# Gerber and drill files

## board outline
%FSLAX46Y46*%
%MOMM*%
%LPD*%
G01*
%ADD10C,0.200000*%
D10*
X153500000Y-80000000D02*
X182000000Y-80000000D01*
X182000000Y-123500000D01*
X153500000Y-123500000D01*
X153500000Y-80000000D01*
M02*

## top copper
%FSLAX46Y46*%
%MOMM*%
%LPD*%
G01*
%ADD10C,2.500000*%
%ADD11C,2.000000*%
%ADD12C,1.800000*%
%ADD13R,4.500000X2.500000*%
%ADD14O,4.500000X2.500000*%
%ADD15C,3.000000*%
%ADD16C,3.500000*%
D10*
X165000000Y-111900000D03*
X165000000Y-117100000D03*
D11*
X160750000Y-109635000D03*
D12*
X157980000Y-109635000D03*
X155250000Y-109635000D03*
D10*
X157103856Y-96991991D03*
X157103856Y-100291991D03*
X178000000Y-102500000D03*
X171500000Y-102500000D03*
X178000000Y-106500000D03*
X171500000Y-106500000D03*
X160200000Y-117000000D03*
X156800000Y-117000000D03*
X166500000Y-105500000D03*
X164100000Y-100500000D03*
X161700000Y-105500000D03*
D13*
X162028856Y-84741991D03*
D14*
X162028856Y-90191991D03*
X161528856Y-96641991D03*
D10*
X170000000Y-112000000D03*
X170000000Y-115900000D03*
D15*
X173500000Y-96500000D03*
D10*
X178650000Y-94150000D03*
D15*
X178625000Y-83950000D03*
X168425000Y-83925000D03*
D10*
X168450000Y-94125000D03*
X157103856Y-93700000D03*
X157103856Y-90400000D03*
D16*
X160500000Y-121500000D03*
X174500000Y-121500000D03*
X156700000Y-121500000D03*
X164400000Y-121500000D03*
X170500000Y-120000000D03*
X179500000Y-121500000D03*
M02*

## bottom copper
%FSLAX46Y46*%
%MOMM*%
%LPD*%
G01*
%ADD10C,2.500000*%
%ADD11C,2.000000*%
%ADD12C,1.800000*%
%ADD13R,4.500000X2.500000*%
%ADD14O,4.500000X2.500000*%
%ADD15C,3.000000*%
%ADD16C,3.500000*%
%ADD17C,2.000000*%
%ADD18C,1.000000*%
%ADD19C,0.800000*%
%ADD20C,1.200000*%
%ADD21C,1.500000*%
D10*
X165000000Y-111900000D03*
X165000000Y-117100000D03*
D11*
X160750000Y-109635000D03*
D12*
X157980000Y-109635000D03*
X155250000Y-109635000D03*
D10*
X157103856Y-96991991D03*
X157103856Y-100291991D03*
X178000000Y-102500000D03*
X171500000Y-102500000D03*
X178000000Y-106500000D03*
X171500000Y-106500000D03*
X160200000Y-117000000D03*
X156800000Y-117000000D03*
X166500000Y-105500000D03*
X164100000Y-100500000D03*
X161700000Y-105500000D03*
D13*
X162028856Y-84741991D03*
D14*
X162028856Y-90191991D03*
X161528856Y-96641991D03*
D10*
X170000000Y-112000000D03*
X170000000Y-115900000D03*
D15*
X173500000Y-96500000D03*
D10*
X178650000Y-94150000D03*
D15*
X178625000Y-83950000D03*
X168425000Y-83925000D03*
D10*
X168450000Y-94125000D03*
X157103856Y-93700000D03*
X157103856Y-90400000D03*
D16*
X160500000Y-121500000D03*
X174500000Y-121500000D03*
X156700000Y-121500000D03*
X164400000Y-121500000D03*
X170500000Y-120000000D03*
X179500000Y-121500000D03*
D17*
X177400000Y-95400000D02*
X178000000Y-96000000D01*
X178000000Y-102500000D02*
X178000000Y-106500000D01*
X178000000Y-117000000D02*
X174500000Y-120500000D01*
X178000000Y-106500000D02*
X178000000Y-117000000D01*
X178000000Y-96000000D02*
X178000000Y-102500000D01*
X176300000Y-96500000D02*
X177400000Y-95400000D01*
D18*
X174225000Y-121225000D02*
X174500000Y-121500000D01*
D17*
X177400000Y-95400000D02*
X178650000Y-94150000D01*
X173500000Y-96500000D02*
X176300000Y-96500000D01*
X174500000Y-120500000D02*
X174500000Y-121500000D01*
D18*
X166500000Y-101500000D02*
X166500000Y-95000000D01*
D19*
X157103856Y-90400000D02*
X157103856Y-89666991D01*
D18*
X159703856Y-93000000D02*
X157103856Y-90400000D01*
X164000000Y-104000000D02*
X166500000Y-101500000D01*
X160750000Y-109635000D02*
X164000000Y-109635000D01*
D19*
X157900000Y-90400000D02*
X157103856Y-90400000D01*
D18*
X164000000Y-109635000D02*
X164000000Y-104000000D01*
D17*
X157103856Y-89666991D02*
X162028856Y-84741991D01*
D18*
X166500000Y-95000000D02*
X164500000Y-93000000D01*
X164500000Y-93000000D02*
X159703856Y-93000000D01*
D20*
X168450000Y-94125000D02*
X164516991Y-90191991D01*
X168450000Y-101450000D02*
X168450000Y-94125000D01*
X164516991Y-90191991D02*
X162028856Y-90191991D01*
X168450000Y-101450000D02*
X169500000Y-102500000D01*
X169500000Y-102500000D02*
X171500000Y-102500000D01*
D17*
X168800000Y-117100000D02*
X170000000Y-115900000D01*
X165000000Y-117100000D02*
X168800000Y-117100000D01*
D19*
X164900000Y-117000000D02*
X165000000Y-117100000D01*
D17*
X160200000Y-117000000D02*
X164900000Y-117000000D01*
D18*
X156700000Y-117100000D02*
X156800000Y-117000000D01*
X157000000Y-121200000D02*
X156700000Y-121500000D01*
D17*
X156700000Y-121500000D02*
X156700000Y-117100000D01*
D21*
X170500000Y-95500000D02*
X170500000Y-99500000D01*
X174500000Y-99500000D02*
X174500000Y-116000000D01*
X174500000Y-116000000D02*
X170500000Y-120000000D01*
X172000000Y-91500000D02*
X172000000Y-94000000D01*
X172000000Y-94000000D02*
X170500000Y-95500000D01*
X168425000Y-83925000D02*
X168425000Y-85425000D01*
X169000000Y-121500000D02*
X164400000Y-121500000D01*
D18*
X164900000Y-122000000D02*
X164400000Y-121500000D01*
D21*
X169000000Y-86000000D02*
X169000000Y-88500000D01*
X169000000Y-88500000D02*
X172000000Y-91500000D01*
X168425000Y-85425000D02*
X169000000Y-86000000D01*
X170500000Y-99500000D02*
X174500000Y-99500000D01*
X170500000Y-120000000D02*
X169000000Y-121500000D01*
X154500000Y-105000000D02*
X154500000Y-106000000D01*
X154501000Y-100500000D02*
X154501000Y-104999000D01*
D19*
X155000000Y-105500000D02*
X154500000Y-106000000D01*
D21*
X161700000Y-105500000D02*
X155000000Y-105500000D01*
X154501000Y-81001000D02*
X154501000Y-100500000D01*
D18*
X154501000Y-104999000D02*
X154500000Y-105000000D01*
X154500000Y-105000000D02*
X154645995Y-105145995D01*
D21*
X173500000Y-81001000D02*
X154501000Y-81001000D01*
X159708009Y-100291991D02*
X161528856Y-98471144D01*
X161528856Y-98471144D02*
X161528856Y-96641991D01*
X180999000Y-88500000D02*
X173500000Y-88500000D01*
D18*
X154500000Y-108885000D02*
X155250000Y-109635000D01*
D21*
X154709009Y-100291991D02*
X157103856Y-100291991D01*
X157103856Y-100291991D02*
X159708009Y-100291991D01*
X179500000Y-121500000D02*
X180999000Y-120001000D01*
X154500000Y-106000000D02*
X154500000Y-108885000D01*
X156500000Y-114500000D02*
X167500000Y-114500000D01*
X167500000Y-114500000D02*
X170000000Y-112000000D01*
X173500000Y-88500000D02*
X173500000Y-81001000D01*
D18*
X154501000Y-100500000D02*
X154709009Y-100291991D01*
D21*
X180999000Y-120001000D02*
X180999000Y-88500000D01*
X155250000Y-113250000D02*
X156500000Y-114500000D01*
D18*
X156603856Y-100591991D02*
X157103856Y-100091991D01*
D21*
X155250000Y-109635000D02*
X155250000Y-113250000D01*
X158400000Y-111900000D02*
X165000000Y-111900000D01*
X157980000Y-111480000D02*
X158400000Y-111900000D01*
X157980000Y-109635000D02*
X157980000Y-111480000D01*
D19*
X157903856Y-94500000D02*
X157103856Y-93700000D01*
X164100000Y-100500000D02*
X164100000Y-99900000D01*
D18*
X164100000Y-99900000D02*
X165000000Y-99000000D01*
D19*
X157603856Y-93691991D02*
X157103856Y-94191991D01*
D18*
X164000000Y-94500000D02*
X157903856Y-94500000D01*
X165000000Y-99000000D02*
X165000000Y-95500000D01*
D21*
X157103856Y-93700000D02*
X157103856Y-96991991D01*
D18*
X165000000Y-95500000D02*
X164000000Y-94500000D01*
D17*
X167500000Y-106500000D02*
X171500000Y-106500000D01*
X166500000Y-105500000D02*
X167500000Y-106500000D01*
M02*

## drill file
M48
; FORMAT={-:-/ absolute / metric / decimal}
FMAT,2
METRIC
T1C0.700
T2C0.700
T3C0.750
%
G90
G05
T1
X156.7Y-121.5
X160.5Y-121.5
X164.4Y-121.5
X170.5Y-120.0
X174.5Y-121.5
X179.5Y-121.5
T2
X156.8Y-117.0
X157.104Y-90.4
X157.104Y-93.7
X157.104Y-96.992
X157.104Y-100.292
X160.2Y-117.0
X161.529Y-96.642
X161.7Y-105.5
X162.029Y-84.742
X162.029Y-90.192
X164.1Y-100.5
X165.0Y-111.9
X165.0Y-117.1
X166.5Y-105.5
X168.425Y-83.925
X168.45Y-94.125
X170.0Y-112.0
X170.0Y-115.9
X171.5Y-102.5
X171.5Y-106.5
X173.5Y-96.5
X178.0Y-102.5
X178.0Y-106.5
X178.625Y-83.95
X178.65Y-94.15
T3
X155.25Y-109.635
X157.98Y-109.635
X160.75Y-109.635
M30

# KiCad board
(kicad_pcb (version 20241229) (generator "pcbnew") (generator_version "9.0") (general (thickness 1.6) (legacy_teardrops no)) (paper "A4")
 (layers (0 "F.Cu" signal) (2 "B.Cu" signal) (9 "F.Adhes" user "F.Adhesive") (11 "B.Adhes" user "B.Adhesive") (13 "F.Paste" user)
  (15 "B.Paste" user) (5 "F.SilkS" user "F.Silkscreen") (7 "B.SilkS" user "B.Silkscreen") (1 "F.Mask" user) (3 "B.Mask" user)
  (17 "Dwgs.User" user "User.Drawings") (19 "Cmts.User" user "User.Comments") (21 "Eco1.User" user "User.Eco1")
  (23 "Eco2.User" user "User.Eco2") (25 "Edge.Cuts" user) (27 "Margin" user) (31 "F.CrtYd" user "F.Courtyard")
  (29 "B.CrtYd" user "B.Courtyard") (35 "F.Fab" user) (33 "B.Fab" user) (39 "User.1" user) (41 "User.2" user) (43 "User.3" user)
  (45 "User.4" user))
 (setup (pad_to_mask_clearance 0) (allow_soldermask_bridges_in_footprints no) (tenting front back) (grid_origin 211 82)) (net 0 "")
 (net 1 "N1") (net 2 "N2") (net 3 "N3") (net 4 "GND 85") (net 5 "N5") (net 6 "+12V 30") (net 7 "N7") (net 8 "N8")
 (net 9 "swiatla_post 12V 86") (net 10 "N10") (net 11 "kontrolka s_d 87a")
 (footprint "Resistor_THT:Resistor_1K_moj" (layer "F.Cu") (at 165 112.5 -90)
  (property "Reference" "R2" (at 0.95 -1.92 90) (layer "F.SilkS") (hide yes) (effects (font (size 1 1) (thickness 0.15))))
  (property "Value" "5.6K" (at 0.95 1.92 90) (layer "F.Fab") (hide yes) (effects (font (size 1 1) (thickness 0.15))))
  (pad "1" thru_hole circle (at -0.6 0 270) (size 2.5 2.5) (drill 0.7) (layers "*.Cu" "*.Mask") (remove_unused_layers no) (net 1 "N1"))
  (pad "2" thru_hole circle (at 4.6 0 270) (size 2.5 2.5) (drill 0.7) (layers "*.Cu" "*.Mask") (remove_unused_layers no) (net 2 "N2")))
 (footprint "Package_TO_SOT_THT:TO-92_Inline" (layer "F.Cu") (at 159.25 109.635 180)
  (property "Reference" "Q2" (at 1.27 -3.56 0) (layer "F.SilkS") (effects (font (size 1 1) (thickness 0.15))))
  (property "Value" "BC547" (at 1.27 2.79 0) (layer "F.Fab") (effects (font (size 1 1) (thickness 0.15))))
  (pad "1" thru_hole circle (at -1.5 0 180) (size 2 2) (drill 0.75) (layers "*.Cu" "*.Mask") (remove_unused_layers no) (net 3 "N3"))
  (pad "2" thru_hole circle (at 1.27 0 180) (size 1.8 1.8) (drill 0.75) (layers "*.Cu" "*.Mask") (remove_unused_layers no) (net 1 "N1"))
  (pad "3" thru_hole circle (at 4 0 180) (size 1.8 1.8) (drill 0.75) (layers "*.Cu" "*.Mask") (remove_unused_layers no) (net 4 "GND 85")))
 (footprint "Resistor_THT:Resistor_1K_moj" (layer "F.Cu") (at 157.103856 98.191991 -90)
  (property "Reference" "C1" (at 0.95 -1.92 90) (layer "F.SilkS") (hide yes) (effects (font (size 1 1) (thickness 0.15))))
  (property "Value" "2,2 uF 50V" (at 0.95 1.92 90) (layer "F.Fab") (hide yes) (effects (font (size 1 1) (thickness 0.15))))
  (pad "1" thru_hole circle (at -1.2 0 270) (size 2.5 2.5) (drill 0.7) (layers "*.Cu" "*.Mask") (remove_unused_layers no) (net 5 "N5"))
  (pad "2" thru_hole circle (at 2.1 0 270) (size 2.5 2.5) (drill 0.7) (layers "*.Cu" "*.Mask") (remove_unused_layers no) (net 4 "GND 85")))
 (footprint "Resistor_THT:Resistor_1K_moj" (layer "F.Cu") (at 177 102.5 180)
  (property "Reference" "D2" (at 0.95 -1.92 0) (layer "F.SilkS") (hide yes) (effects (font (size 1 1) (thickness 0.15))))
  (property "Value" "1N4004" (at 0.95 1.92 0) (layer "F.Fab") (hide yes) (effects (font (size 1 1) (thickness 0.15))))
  (pad "1" thru_hole circle (at -1 0 180) (size 2.5 2.5) (drill 0.7) (layers "*.Cu" "*.Mask") (remove_unused_layers no) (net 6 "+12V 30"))
  (pad "2" thru_hole circle (at 5.5 0 180) (size 2.5 2.5) (drill 0.7) (layers "*.Cu" "*.Mask") (remove_unused_layers no) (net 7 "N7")))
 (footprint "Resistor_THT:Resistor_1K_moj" (layer "F.Cu") (at 177 106.5 180)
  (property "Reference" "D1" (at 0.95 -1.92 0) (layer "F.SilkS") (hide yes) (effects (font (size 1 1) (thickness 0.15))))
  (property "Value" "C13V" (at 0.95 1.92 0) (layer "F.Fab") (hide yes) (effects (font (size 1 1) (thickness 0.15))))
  (pad "1" thru_hole circle (at -1 0 180) (size 2.5 2.5) (drill 0.7) (layers "*.Cu" "*.Mask") (remove_unused_layers no) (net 6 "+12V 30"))
  (pad "2" thru_hole circle (at 5.5 0 180) (size 2.5 2.5) (drill 0.7) (layers "*.Cu" "*.Mask") (remove_unused_layers no) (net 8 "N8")))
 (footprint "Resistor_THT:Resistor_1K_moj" (layer "F.Cu") (at 158 117)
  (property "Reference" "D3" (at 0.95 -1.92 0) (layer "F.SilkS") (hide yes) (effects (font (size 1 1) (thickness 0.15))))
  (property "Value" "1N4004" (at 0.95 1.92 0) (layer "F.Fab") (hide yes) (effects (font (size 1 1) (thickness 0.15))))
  (pad "" thru_hole circle (at 2.2 0) (size 2.5 2.5) (drill 0.7) (layers "*.Cu" "*.Mask") (remove_unused_layers no) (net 2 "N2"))
  (pad "1" thru_hole circle (at -1.2 0) (size 2.5 2.5) (drill 0.7) (layers "*.Cu" "*.Mask") (remove_unused_layers no)
   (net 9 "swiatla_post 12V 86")))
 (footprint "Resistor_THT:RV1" (layer "F.Cu") (at 164 103.5 -90)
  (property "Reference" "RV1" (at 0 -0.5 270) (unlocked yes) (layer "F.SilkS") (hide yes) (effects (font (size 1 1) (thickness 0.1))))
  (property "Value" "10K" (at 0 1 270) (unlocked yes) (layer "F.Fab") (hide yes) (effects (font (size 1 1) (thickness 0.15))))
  (pad "1" thru_hole circle (at 2 -2.5 270) (size 2.5 2.5) (drill 0.7) (layers "*.Cu" "*.Mask") (remove_unused_layers no) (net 8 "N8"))
  (pad "2" thru_hole circle (at -3 -0.1 270) (size 2.5 2.5) (drill 0.7) (layers "*.Cu" "*.Mask") (remove_unused_layers no) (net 5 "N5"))
  (pad "3" thru_hole circle (at 2 2.3 270) (size 2.5 2.5) (drill 0.7) (layers "*.Cu" "*.Mask") (remove_unused_layers no) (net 4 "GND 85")))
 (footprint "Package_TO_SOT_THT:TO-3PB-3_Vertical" (layer "F.Cu") (at 162.028856 84.741991 -90)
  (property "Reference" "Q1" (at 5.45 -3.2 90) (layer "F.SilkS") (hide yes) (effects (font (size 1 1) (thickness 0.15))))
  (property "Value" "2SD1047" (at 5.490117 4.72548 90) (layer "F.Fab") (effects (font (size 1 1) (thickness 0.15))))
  (pad "1" thru_hole rect (at 0 0 270) (size 2.5 4.5) (drill 0.7) (layers "*.Cu" "*.Mask") (remove_unused_layers no) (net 3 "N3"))
  (pad "2" thru_hole oval (at 5.45 0 270) (size 2.5 4.5) (drill 0.7) (layers "*.Cu" "*.Mask") (remove_unused_layers no) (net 7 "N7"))
  (pad "3" thru_hole oval (at 11.9 0.5 270) (size 2.5 4.5) (drill 0.7) (layers "*.Cu" "*.Mask") (remove_unused_layers no) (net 4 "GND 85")))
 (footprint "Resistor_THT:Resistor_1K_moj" (layer "F.Cu") (at 170 113 -90)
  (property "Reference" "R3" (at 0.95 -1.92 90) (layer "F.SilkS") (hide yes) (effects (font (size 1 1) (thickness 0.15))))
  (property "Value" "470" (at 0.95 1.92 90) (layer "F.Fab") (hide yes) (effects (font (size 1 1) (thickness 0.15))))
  (pad "1" thru_hole circle (at -1 0 270) (size 2.5 2.5) (drill 0.7) (layers "*.Cu" "*.Mask") (remove_unused_layers no) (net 4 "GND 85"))
  (pad "2" thru_hole circle (at 2.9 0 270) (size 2.5 2.5) (drill 0.7) (layers "*.Cu" "*.Mask") (remove_unused_layers no) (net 2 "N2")))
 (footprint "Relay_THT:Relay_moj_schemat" (layer "F.Cu") (at 173.5 97.1 90)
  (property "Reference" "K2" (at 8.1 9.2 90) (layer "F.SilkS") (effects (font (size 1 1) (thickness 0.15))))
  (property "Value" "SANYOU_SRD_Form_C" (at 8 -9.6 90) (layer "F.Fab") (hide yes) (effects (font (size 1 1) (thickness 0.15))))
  (pad "1" thru_hole circle (at 0.6 0 180) (size 3 3) (drill 0.7) (layers "*.Cu" "*.Mask") (remove_unused_layers no) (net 6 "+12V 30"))
  (pad "2" thru_hole circle (at 2.95 5.15 180) (size 2.5 2.5) (drill 0.7) (layers "*.Cu" "*.Mask") (remove_unused_layers no)
   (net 6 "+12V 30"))
  (pad "3" thru_hole circle (at 13.15 5.125 180) (size 3 3) (drill 0.7) (layers "*.Cu" "*.Mask") (remove_unused_layers no) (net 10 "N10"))
  (pad "4" thru_hole circle (at 13.175 -5.075 180) (size 3 3) (drill 0.7) (layers "*.Cu" "*.Mask") (remove_unused_layers no)
   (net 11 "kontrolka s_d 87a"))
  (pad "5" thru_hole circle (at 2.975 -5.05 180) (size 2.5 2.5) (drill 0.7) (layers "*.Cu" "*.Mask") (remove_unused_layers no) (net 7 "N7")))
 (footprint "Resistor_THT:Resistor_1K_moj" (layer "F.Cu") (at 157.103856 92.5 90)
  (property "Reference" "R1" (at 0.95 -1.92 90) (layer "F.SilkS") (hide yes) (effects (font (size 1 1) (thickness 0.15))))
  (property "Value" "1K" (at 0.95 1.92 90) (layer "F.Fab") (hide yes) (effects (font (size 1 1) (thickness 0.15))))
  (pad "1" thru_hole circle (at -1.2 0 90) (size 2.5 2.5) (drill 0.7) (layers "*.Cu" "*.Mask") (remove_unused_layers no) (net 5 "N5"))
  (pad "2" thru_hole circle (at 2.1 0 90) (size 2.5 2.5) (drill 0.7) (layers "*.Cu" "*.Mask") (remove_unused_layers no) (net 3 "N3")))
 (gr_rect (start 153.5 80) (end 182 123.5) (stroke (width 0.2) (type solid)) (fill no) (layer "Edge.Cuts"))
 (via (at 160.5 121.5) (size 3.5) (drill 0.7) (layers "F.Cu" "B.Cu") (free yes) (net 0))
 (via (at 174.5 121.5) (size 3.5) (drill 0.7) (layers "F.Cu" "B.Cu") (free yes) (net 6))
 (segment (start 177.4 95.4) (end 178 96) (width 2) (layer "B.Cu") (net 6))
 (segment (start 178 102.5) (end 178 106.5) (width 2) (layer "B.Cu") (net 6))
 (segment (start 178 117) (end 174.5 120.5) (width 2) (layer "B.Cu") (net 6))
 (segment (start 178 106.5) (end 178 117) (width 2) (layer "B.Cu") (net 6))
 (segment (start 178 96) (end 178 102.5) (width 2) (layer "B.Cu") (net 6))
 (segment (start 176.3 96.5) (end 177.4 95.4) (width 2) (layer "B.Cu") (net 6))
 (segment (start 174.225 121.225) (end 174.5 121.5) (width 1) (layer "B.Cu") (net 6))
 (segment (start 177.4 95.4) (end 178.65 94.15) (width 2) (layer "B.Cu") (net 6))
 (segment (start 173.5 96.5) (end 176.3 96.5) (width 2) (layer "B.Cu") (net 6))
 (segment (start 174.5 120.5) (end 174.5 121.5) (width 2) (layer "B.Cu") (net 6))
 (segment (start 166.5 101.5) (end 166.5 95) (width 1) (layer "B.Cu") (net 3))
 (segment (start 157.103856 90.4) (end 157.103856 89.666991) (width 0.8) (layer "B.Cu") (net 3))
 (segment (start 159.703856 93) (end 157.103856 90.4) (width 1) (layer "B.Cu") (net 3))
 (segment (start 164 104) (end 166.5 101.5) (width 1) (layer "B.Cu") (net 3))
 (segment (start 160.75 109.635) (end 164 109.635) (width 1) (layer "B.Cu") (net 3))
 (segment (start 157.9 90.4) (end 157.103856 90.4) (width 0.8) (layer "B.Cu") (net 3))
 (segment (start 164 109.635) (end 164 104) (width 1) (layer "B.Cu") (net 3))
 (segment (start 157.103856 89.666991) (end 162.028856 84.741991) (width 2) (layer "B.Cu") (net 3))
 (segment (start 166.5 95) (end 164.5 93) (width 1) (layer "B.Cu") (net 3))
 (segment (start 164.5 93) (end 159.703856 93) (width 1) (layer "B.Cu") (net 3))
 (segment (start 168.45 94.125) (end 164.516991 90.191991) (width 1.2) (layer "B.Cu") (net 7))
 (segment (start 168.45 101.45) (end 168.45 94.125) (width 1.2) (layer "B.Cu") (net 7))
 (segment (start 164.516991 90.191991) (end 162.028856 90.191991) (width 1.2) (layer "B.Cu") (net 7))
 (segment (start 168.45 101.45) (end 169.5 102.5) (width 1.2) (layer "B.Cu") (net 7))
 (segment (start 169.5 102.5) (end 171.5 102.5) (width 1.2) (layer "B.Cu") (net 7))
 (segment (start 168.8 117.1) (end 170 115.9) (width 2) (layer "B.Cu") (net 2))
 (segment (start 165 117.1) (end 168.8 117.1) (width 2) (layer "B.Cu") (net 2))
 (segment (start 164.9 117) (end 165 117.1) (width 0.8) (layer "B.Cu") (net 2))
 (segment (start 160.2 117) (end 164.9 117) (width 2) (layer "B.Cu") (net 2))
 (via (at 156.7 121.5) (size 3.5) (drill 0.7) (layers "F.Cu" "B.Cu") (free yes) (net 9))
 (segment (start 156.7 117.1) (end 156.8 117) (width 1) (layer "B.Cu") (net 9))
 (segment (start 157 121.2) (end 156.7 121.5) (width 1) (layer "B.Cu") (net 9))
 (segment (start 156.7 121.5) (end 156.7 117.1) (width 2) (layer "B.Cu") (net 9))
 (via (at 164.4 121.5) (size 3.5) (drill 0.7) (layers "F.Cu" "B.Cu") (free yes) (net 11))
 (via (at 170.5 120) (size 3.5) (drill 0.7) (layers "F.Cu" "B.Cu") (free yes) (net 11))
 (segment (start 170.5 95.5) (end 170.5 99.5) (width 1.5) (layer "B.Cu") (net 11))
 (segment (start 174.5 99.5) (end 174.5 116) (width 1.5) (layer "B.Cu") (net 11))
 (segment (start 174.5 116) (end 170.5 120) (width 1.5) (layer "B.Cu") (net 11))
 (segment (start 172 91.5) (end 172 94) (width 1.5) (layer "B.Cu") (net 11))
 (segment (start 172 94) (end 170.5 95.5) (width 1.5) (layer "B.Cu") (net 11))
 (segment (start 168.425 83.925) (end 168.425 85.425) (width 1.5) (layer "B.Cu") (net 11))
 (segment (start 169 121.5) (end 164.4 121.5) (width 1.5) (layer "B.Cu") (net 11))
 (segment (start 164.9 122) (end 164.4 121.5) (width 1) (layer "B.Cu") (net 11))
 (segment (start 169 86) (end 169 88.5) (width 1.5) (layer "B.Cu") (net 11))
 (segment (start 169 88.5) (end 172 91.5) (width 1.5) (layer "B.Cu") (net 11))
 (segment (start 168.425 85.425) (end 169 86) (width 1.5) (layer "B.Cu") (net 11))
 (segment (start 170.5 99.5) (end 174.5 99.5) (width 1.5) (layer "B.Cu") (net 11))
 (segment (start 170.5 120) (end 169 121.5) (width 1.5) (layer "B.Cu") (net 11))
 (via (at 179.5 121.5) (size 3.5) (drill 0.7) (layers "F.Cu" "B.Cu") (free yes) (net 4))
 (segment (start 154.5 105) (end 154.5 106) (width 1.5) (layer "B.Cu") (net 4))
 (segment (start 154.501 100.5) (end 154.501 104.999) (width 1.5) (layer "B.Cu") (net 4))
 (segment (start 155 105.5) (end 154.5 106) (width 0.8) (layer "B.Cu") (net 4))
 (segment (start 161.7 105.5) (end 155 105.5) (width 1.5) (layer "B.Cu") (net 4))
 (segment (start 154.501 81.001) (end 154.501 100.5) (width 1.5) (layer "B.Cu") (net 4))
 (segment (start 154.501 104.999) (end 154.5 105) (width 1) (layer "B.Cu") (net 4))
 (segment (start 154.5 105) (end 154.645995 105.145995) (width 1) (layer "B.Cu") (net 4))
 (segment (start 173.5 81.001) (end 154.501 81.001) (width 1.5) (layer "B.Cu") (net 4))
 (segment (start 159.708009 100.291991) (end 161.528856 98.471144) (width 1.5) (layer "B.Cu") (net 4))
 (segment (start 161.528856 98.471144) (end 161.528856 96.641991) (width 1.5) (layer "B.Cu") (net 4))
 (segment (start 180.999 88.5) (end 173.5 88.5) (width 1.5) (layer "B.Cu") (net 4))
 (segment (start 154.5 108.885) (end 155.25 109.635) (width 1) (layer "B.Cu") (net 4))
 (segment (start 154.709009 100.291991) (end 157.103856 100.291991) (width 1.5) (layer "B.Cu") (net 4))
 (segment (start 157.103856 100.291991) (end 159.708009 100.291991) (width 1.5) (layer "B.Cu") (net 4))
 (segment (start 179.5 121.5) (end 180.999 120.001) (width 1.5) (layer "B.Cu") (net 4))
 (segment (start 154.5 106) (end 154.5 108.885) (width 1.5) (layer "B.Cu") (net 4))
 (segment (start 156.5 114.5) (end 167.5 114.5) (width 1.5) (layer "B.Cu") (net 4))
 (segment (start 167.5 114.5) (end 170 112) (width 1.5) (layer "B.Cu") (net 4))
 (segment (start 173.5 88.5) (end 173.5 81.001) (width 1.5) (layer "B.Cu") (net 4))
 (segment (start 154.501 100.5) (end 154.709009 100.291991) (width 1) (layer "B.Cu") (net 4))
 (segment (start 180.999 120.001) (end 180.999 88.5) (width 1.5) (layer "B.Cu") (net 4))
 (segment (start 155.25 113.25) (end 156.5 114.5) (width 1.5) (layer "B.Cu") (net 4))
 (segment (start 156.603856 100.591991) (end 157.103856 100.091991) (width 1) (layer "B.Cu") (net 4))
 (segment (start 155.25 109.635) (end 155.25 113.25) (width 1.5) (layer "B.Cu") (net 4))
 (segment (start 158.4 111.9) (end 165 111.9) (width 1.5) (layer "B.Cu") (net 1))
 (segment (start 157.98 111.48) (end 158.4 111.9) (width 1.5) (layer "B.Cu") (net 1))
 (segment (start 157.98 109.635) (end 157.98 111.48) (width 1.5) (layer "B.Cu") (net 1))
 (segment (start 157.903856 94.5) (end 157.103856 93.7) (width 0.8) (layer "B.Cu") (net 5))
 (segment (start 164.1 100.5) (end 164.1 99.9) (width 0.8) (layer "B.Cu") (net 5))
 (segment (start 164.1 99.9) (end 165 99) (width 1) (layer "B.Cu") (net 5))
 (segment (start 157.603856 93.691991) (end 157.103856 94.191991) (width 0.8) (layer "B.Cu") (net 5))
 (segment (start 164 94.5) (end 157.903856 94.5) (width 1) (layer "B.Cu") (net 5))
 (segment (start 165 99) (end 165 95.5) (width 1) (layer "B.Cu") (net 5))
 (segment (start 157.103856 93.7) (end 157.103856 96.991991) (width 1.5) (layer "B.Cu") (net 5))
 (segment (start 165 95.5) (end 164 94.5) (width 1) (layer "B.Cu") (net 5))
 (segment (start 167.5 106.5) (end 171.5 106.5) (width 2) (layer "B.Cu") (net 8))
 (segment (start 166.5 105.5) (end 167.5 106.5) (width 2) (layer "B.Cu") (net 8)))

